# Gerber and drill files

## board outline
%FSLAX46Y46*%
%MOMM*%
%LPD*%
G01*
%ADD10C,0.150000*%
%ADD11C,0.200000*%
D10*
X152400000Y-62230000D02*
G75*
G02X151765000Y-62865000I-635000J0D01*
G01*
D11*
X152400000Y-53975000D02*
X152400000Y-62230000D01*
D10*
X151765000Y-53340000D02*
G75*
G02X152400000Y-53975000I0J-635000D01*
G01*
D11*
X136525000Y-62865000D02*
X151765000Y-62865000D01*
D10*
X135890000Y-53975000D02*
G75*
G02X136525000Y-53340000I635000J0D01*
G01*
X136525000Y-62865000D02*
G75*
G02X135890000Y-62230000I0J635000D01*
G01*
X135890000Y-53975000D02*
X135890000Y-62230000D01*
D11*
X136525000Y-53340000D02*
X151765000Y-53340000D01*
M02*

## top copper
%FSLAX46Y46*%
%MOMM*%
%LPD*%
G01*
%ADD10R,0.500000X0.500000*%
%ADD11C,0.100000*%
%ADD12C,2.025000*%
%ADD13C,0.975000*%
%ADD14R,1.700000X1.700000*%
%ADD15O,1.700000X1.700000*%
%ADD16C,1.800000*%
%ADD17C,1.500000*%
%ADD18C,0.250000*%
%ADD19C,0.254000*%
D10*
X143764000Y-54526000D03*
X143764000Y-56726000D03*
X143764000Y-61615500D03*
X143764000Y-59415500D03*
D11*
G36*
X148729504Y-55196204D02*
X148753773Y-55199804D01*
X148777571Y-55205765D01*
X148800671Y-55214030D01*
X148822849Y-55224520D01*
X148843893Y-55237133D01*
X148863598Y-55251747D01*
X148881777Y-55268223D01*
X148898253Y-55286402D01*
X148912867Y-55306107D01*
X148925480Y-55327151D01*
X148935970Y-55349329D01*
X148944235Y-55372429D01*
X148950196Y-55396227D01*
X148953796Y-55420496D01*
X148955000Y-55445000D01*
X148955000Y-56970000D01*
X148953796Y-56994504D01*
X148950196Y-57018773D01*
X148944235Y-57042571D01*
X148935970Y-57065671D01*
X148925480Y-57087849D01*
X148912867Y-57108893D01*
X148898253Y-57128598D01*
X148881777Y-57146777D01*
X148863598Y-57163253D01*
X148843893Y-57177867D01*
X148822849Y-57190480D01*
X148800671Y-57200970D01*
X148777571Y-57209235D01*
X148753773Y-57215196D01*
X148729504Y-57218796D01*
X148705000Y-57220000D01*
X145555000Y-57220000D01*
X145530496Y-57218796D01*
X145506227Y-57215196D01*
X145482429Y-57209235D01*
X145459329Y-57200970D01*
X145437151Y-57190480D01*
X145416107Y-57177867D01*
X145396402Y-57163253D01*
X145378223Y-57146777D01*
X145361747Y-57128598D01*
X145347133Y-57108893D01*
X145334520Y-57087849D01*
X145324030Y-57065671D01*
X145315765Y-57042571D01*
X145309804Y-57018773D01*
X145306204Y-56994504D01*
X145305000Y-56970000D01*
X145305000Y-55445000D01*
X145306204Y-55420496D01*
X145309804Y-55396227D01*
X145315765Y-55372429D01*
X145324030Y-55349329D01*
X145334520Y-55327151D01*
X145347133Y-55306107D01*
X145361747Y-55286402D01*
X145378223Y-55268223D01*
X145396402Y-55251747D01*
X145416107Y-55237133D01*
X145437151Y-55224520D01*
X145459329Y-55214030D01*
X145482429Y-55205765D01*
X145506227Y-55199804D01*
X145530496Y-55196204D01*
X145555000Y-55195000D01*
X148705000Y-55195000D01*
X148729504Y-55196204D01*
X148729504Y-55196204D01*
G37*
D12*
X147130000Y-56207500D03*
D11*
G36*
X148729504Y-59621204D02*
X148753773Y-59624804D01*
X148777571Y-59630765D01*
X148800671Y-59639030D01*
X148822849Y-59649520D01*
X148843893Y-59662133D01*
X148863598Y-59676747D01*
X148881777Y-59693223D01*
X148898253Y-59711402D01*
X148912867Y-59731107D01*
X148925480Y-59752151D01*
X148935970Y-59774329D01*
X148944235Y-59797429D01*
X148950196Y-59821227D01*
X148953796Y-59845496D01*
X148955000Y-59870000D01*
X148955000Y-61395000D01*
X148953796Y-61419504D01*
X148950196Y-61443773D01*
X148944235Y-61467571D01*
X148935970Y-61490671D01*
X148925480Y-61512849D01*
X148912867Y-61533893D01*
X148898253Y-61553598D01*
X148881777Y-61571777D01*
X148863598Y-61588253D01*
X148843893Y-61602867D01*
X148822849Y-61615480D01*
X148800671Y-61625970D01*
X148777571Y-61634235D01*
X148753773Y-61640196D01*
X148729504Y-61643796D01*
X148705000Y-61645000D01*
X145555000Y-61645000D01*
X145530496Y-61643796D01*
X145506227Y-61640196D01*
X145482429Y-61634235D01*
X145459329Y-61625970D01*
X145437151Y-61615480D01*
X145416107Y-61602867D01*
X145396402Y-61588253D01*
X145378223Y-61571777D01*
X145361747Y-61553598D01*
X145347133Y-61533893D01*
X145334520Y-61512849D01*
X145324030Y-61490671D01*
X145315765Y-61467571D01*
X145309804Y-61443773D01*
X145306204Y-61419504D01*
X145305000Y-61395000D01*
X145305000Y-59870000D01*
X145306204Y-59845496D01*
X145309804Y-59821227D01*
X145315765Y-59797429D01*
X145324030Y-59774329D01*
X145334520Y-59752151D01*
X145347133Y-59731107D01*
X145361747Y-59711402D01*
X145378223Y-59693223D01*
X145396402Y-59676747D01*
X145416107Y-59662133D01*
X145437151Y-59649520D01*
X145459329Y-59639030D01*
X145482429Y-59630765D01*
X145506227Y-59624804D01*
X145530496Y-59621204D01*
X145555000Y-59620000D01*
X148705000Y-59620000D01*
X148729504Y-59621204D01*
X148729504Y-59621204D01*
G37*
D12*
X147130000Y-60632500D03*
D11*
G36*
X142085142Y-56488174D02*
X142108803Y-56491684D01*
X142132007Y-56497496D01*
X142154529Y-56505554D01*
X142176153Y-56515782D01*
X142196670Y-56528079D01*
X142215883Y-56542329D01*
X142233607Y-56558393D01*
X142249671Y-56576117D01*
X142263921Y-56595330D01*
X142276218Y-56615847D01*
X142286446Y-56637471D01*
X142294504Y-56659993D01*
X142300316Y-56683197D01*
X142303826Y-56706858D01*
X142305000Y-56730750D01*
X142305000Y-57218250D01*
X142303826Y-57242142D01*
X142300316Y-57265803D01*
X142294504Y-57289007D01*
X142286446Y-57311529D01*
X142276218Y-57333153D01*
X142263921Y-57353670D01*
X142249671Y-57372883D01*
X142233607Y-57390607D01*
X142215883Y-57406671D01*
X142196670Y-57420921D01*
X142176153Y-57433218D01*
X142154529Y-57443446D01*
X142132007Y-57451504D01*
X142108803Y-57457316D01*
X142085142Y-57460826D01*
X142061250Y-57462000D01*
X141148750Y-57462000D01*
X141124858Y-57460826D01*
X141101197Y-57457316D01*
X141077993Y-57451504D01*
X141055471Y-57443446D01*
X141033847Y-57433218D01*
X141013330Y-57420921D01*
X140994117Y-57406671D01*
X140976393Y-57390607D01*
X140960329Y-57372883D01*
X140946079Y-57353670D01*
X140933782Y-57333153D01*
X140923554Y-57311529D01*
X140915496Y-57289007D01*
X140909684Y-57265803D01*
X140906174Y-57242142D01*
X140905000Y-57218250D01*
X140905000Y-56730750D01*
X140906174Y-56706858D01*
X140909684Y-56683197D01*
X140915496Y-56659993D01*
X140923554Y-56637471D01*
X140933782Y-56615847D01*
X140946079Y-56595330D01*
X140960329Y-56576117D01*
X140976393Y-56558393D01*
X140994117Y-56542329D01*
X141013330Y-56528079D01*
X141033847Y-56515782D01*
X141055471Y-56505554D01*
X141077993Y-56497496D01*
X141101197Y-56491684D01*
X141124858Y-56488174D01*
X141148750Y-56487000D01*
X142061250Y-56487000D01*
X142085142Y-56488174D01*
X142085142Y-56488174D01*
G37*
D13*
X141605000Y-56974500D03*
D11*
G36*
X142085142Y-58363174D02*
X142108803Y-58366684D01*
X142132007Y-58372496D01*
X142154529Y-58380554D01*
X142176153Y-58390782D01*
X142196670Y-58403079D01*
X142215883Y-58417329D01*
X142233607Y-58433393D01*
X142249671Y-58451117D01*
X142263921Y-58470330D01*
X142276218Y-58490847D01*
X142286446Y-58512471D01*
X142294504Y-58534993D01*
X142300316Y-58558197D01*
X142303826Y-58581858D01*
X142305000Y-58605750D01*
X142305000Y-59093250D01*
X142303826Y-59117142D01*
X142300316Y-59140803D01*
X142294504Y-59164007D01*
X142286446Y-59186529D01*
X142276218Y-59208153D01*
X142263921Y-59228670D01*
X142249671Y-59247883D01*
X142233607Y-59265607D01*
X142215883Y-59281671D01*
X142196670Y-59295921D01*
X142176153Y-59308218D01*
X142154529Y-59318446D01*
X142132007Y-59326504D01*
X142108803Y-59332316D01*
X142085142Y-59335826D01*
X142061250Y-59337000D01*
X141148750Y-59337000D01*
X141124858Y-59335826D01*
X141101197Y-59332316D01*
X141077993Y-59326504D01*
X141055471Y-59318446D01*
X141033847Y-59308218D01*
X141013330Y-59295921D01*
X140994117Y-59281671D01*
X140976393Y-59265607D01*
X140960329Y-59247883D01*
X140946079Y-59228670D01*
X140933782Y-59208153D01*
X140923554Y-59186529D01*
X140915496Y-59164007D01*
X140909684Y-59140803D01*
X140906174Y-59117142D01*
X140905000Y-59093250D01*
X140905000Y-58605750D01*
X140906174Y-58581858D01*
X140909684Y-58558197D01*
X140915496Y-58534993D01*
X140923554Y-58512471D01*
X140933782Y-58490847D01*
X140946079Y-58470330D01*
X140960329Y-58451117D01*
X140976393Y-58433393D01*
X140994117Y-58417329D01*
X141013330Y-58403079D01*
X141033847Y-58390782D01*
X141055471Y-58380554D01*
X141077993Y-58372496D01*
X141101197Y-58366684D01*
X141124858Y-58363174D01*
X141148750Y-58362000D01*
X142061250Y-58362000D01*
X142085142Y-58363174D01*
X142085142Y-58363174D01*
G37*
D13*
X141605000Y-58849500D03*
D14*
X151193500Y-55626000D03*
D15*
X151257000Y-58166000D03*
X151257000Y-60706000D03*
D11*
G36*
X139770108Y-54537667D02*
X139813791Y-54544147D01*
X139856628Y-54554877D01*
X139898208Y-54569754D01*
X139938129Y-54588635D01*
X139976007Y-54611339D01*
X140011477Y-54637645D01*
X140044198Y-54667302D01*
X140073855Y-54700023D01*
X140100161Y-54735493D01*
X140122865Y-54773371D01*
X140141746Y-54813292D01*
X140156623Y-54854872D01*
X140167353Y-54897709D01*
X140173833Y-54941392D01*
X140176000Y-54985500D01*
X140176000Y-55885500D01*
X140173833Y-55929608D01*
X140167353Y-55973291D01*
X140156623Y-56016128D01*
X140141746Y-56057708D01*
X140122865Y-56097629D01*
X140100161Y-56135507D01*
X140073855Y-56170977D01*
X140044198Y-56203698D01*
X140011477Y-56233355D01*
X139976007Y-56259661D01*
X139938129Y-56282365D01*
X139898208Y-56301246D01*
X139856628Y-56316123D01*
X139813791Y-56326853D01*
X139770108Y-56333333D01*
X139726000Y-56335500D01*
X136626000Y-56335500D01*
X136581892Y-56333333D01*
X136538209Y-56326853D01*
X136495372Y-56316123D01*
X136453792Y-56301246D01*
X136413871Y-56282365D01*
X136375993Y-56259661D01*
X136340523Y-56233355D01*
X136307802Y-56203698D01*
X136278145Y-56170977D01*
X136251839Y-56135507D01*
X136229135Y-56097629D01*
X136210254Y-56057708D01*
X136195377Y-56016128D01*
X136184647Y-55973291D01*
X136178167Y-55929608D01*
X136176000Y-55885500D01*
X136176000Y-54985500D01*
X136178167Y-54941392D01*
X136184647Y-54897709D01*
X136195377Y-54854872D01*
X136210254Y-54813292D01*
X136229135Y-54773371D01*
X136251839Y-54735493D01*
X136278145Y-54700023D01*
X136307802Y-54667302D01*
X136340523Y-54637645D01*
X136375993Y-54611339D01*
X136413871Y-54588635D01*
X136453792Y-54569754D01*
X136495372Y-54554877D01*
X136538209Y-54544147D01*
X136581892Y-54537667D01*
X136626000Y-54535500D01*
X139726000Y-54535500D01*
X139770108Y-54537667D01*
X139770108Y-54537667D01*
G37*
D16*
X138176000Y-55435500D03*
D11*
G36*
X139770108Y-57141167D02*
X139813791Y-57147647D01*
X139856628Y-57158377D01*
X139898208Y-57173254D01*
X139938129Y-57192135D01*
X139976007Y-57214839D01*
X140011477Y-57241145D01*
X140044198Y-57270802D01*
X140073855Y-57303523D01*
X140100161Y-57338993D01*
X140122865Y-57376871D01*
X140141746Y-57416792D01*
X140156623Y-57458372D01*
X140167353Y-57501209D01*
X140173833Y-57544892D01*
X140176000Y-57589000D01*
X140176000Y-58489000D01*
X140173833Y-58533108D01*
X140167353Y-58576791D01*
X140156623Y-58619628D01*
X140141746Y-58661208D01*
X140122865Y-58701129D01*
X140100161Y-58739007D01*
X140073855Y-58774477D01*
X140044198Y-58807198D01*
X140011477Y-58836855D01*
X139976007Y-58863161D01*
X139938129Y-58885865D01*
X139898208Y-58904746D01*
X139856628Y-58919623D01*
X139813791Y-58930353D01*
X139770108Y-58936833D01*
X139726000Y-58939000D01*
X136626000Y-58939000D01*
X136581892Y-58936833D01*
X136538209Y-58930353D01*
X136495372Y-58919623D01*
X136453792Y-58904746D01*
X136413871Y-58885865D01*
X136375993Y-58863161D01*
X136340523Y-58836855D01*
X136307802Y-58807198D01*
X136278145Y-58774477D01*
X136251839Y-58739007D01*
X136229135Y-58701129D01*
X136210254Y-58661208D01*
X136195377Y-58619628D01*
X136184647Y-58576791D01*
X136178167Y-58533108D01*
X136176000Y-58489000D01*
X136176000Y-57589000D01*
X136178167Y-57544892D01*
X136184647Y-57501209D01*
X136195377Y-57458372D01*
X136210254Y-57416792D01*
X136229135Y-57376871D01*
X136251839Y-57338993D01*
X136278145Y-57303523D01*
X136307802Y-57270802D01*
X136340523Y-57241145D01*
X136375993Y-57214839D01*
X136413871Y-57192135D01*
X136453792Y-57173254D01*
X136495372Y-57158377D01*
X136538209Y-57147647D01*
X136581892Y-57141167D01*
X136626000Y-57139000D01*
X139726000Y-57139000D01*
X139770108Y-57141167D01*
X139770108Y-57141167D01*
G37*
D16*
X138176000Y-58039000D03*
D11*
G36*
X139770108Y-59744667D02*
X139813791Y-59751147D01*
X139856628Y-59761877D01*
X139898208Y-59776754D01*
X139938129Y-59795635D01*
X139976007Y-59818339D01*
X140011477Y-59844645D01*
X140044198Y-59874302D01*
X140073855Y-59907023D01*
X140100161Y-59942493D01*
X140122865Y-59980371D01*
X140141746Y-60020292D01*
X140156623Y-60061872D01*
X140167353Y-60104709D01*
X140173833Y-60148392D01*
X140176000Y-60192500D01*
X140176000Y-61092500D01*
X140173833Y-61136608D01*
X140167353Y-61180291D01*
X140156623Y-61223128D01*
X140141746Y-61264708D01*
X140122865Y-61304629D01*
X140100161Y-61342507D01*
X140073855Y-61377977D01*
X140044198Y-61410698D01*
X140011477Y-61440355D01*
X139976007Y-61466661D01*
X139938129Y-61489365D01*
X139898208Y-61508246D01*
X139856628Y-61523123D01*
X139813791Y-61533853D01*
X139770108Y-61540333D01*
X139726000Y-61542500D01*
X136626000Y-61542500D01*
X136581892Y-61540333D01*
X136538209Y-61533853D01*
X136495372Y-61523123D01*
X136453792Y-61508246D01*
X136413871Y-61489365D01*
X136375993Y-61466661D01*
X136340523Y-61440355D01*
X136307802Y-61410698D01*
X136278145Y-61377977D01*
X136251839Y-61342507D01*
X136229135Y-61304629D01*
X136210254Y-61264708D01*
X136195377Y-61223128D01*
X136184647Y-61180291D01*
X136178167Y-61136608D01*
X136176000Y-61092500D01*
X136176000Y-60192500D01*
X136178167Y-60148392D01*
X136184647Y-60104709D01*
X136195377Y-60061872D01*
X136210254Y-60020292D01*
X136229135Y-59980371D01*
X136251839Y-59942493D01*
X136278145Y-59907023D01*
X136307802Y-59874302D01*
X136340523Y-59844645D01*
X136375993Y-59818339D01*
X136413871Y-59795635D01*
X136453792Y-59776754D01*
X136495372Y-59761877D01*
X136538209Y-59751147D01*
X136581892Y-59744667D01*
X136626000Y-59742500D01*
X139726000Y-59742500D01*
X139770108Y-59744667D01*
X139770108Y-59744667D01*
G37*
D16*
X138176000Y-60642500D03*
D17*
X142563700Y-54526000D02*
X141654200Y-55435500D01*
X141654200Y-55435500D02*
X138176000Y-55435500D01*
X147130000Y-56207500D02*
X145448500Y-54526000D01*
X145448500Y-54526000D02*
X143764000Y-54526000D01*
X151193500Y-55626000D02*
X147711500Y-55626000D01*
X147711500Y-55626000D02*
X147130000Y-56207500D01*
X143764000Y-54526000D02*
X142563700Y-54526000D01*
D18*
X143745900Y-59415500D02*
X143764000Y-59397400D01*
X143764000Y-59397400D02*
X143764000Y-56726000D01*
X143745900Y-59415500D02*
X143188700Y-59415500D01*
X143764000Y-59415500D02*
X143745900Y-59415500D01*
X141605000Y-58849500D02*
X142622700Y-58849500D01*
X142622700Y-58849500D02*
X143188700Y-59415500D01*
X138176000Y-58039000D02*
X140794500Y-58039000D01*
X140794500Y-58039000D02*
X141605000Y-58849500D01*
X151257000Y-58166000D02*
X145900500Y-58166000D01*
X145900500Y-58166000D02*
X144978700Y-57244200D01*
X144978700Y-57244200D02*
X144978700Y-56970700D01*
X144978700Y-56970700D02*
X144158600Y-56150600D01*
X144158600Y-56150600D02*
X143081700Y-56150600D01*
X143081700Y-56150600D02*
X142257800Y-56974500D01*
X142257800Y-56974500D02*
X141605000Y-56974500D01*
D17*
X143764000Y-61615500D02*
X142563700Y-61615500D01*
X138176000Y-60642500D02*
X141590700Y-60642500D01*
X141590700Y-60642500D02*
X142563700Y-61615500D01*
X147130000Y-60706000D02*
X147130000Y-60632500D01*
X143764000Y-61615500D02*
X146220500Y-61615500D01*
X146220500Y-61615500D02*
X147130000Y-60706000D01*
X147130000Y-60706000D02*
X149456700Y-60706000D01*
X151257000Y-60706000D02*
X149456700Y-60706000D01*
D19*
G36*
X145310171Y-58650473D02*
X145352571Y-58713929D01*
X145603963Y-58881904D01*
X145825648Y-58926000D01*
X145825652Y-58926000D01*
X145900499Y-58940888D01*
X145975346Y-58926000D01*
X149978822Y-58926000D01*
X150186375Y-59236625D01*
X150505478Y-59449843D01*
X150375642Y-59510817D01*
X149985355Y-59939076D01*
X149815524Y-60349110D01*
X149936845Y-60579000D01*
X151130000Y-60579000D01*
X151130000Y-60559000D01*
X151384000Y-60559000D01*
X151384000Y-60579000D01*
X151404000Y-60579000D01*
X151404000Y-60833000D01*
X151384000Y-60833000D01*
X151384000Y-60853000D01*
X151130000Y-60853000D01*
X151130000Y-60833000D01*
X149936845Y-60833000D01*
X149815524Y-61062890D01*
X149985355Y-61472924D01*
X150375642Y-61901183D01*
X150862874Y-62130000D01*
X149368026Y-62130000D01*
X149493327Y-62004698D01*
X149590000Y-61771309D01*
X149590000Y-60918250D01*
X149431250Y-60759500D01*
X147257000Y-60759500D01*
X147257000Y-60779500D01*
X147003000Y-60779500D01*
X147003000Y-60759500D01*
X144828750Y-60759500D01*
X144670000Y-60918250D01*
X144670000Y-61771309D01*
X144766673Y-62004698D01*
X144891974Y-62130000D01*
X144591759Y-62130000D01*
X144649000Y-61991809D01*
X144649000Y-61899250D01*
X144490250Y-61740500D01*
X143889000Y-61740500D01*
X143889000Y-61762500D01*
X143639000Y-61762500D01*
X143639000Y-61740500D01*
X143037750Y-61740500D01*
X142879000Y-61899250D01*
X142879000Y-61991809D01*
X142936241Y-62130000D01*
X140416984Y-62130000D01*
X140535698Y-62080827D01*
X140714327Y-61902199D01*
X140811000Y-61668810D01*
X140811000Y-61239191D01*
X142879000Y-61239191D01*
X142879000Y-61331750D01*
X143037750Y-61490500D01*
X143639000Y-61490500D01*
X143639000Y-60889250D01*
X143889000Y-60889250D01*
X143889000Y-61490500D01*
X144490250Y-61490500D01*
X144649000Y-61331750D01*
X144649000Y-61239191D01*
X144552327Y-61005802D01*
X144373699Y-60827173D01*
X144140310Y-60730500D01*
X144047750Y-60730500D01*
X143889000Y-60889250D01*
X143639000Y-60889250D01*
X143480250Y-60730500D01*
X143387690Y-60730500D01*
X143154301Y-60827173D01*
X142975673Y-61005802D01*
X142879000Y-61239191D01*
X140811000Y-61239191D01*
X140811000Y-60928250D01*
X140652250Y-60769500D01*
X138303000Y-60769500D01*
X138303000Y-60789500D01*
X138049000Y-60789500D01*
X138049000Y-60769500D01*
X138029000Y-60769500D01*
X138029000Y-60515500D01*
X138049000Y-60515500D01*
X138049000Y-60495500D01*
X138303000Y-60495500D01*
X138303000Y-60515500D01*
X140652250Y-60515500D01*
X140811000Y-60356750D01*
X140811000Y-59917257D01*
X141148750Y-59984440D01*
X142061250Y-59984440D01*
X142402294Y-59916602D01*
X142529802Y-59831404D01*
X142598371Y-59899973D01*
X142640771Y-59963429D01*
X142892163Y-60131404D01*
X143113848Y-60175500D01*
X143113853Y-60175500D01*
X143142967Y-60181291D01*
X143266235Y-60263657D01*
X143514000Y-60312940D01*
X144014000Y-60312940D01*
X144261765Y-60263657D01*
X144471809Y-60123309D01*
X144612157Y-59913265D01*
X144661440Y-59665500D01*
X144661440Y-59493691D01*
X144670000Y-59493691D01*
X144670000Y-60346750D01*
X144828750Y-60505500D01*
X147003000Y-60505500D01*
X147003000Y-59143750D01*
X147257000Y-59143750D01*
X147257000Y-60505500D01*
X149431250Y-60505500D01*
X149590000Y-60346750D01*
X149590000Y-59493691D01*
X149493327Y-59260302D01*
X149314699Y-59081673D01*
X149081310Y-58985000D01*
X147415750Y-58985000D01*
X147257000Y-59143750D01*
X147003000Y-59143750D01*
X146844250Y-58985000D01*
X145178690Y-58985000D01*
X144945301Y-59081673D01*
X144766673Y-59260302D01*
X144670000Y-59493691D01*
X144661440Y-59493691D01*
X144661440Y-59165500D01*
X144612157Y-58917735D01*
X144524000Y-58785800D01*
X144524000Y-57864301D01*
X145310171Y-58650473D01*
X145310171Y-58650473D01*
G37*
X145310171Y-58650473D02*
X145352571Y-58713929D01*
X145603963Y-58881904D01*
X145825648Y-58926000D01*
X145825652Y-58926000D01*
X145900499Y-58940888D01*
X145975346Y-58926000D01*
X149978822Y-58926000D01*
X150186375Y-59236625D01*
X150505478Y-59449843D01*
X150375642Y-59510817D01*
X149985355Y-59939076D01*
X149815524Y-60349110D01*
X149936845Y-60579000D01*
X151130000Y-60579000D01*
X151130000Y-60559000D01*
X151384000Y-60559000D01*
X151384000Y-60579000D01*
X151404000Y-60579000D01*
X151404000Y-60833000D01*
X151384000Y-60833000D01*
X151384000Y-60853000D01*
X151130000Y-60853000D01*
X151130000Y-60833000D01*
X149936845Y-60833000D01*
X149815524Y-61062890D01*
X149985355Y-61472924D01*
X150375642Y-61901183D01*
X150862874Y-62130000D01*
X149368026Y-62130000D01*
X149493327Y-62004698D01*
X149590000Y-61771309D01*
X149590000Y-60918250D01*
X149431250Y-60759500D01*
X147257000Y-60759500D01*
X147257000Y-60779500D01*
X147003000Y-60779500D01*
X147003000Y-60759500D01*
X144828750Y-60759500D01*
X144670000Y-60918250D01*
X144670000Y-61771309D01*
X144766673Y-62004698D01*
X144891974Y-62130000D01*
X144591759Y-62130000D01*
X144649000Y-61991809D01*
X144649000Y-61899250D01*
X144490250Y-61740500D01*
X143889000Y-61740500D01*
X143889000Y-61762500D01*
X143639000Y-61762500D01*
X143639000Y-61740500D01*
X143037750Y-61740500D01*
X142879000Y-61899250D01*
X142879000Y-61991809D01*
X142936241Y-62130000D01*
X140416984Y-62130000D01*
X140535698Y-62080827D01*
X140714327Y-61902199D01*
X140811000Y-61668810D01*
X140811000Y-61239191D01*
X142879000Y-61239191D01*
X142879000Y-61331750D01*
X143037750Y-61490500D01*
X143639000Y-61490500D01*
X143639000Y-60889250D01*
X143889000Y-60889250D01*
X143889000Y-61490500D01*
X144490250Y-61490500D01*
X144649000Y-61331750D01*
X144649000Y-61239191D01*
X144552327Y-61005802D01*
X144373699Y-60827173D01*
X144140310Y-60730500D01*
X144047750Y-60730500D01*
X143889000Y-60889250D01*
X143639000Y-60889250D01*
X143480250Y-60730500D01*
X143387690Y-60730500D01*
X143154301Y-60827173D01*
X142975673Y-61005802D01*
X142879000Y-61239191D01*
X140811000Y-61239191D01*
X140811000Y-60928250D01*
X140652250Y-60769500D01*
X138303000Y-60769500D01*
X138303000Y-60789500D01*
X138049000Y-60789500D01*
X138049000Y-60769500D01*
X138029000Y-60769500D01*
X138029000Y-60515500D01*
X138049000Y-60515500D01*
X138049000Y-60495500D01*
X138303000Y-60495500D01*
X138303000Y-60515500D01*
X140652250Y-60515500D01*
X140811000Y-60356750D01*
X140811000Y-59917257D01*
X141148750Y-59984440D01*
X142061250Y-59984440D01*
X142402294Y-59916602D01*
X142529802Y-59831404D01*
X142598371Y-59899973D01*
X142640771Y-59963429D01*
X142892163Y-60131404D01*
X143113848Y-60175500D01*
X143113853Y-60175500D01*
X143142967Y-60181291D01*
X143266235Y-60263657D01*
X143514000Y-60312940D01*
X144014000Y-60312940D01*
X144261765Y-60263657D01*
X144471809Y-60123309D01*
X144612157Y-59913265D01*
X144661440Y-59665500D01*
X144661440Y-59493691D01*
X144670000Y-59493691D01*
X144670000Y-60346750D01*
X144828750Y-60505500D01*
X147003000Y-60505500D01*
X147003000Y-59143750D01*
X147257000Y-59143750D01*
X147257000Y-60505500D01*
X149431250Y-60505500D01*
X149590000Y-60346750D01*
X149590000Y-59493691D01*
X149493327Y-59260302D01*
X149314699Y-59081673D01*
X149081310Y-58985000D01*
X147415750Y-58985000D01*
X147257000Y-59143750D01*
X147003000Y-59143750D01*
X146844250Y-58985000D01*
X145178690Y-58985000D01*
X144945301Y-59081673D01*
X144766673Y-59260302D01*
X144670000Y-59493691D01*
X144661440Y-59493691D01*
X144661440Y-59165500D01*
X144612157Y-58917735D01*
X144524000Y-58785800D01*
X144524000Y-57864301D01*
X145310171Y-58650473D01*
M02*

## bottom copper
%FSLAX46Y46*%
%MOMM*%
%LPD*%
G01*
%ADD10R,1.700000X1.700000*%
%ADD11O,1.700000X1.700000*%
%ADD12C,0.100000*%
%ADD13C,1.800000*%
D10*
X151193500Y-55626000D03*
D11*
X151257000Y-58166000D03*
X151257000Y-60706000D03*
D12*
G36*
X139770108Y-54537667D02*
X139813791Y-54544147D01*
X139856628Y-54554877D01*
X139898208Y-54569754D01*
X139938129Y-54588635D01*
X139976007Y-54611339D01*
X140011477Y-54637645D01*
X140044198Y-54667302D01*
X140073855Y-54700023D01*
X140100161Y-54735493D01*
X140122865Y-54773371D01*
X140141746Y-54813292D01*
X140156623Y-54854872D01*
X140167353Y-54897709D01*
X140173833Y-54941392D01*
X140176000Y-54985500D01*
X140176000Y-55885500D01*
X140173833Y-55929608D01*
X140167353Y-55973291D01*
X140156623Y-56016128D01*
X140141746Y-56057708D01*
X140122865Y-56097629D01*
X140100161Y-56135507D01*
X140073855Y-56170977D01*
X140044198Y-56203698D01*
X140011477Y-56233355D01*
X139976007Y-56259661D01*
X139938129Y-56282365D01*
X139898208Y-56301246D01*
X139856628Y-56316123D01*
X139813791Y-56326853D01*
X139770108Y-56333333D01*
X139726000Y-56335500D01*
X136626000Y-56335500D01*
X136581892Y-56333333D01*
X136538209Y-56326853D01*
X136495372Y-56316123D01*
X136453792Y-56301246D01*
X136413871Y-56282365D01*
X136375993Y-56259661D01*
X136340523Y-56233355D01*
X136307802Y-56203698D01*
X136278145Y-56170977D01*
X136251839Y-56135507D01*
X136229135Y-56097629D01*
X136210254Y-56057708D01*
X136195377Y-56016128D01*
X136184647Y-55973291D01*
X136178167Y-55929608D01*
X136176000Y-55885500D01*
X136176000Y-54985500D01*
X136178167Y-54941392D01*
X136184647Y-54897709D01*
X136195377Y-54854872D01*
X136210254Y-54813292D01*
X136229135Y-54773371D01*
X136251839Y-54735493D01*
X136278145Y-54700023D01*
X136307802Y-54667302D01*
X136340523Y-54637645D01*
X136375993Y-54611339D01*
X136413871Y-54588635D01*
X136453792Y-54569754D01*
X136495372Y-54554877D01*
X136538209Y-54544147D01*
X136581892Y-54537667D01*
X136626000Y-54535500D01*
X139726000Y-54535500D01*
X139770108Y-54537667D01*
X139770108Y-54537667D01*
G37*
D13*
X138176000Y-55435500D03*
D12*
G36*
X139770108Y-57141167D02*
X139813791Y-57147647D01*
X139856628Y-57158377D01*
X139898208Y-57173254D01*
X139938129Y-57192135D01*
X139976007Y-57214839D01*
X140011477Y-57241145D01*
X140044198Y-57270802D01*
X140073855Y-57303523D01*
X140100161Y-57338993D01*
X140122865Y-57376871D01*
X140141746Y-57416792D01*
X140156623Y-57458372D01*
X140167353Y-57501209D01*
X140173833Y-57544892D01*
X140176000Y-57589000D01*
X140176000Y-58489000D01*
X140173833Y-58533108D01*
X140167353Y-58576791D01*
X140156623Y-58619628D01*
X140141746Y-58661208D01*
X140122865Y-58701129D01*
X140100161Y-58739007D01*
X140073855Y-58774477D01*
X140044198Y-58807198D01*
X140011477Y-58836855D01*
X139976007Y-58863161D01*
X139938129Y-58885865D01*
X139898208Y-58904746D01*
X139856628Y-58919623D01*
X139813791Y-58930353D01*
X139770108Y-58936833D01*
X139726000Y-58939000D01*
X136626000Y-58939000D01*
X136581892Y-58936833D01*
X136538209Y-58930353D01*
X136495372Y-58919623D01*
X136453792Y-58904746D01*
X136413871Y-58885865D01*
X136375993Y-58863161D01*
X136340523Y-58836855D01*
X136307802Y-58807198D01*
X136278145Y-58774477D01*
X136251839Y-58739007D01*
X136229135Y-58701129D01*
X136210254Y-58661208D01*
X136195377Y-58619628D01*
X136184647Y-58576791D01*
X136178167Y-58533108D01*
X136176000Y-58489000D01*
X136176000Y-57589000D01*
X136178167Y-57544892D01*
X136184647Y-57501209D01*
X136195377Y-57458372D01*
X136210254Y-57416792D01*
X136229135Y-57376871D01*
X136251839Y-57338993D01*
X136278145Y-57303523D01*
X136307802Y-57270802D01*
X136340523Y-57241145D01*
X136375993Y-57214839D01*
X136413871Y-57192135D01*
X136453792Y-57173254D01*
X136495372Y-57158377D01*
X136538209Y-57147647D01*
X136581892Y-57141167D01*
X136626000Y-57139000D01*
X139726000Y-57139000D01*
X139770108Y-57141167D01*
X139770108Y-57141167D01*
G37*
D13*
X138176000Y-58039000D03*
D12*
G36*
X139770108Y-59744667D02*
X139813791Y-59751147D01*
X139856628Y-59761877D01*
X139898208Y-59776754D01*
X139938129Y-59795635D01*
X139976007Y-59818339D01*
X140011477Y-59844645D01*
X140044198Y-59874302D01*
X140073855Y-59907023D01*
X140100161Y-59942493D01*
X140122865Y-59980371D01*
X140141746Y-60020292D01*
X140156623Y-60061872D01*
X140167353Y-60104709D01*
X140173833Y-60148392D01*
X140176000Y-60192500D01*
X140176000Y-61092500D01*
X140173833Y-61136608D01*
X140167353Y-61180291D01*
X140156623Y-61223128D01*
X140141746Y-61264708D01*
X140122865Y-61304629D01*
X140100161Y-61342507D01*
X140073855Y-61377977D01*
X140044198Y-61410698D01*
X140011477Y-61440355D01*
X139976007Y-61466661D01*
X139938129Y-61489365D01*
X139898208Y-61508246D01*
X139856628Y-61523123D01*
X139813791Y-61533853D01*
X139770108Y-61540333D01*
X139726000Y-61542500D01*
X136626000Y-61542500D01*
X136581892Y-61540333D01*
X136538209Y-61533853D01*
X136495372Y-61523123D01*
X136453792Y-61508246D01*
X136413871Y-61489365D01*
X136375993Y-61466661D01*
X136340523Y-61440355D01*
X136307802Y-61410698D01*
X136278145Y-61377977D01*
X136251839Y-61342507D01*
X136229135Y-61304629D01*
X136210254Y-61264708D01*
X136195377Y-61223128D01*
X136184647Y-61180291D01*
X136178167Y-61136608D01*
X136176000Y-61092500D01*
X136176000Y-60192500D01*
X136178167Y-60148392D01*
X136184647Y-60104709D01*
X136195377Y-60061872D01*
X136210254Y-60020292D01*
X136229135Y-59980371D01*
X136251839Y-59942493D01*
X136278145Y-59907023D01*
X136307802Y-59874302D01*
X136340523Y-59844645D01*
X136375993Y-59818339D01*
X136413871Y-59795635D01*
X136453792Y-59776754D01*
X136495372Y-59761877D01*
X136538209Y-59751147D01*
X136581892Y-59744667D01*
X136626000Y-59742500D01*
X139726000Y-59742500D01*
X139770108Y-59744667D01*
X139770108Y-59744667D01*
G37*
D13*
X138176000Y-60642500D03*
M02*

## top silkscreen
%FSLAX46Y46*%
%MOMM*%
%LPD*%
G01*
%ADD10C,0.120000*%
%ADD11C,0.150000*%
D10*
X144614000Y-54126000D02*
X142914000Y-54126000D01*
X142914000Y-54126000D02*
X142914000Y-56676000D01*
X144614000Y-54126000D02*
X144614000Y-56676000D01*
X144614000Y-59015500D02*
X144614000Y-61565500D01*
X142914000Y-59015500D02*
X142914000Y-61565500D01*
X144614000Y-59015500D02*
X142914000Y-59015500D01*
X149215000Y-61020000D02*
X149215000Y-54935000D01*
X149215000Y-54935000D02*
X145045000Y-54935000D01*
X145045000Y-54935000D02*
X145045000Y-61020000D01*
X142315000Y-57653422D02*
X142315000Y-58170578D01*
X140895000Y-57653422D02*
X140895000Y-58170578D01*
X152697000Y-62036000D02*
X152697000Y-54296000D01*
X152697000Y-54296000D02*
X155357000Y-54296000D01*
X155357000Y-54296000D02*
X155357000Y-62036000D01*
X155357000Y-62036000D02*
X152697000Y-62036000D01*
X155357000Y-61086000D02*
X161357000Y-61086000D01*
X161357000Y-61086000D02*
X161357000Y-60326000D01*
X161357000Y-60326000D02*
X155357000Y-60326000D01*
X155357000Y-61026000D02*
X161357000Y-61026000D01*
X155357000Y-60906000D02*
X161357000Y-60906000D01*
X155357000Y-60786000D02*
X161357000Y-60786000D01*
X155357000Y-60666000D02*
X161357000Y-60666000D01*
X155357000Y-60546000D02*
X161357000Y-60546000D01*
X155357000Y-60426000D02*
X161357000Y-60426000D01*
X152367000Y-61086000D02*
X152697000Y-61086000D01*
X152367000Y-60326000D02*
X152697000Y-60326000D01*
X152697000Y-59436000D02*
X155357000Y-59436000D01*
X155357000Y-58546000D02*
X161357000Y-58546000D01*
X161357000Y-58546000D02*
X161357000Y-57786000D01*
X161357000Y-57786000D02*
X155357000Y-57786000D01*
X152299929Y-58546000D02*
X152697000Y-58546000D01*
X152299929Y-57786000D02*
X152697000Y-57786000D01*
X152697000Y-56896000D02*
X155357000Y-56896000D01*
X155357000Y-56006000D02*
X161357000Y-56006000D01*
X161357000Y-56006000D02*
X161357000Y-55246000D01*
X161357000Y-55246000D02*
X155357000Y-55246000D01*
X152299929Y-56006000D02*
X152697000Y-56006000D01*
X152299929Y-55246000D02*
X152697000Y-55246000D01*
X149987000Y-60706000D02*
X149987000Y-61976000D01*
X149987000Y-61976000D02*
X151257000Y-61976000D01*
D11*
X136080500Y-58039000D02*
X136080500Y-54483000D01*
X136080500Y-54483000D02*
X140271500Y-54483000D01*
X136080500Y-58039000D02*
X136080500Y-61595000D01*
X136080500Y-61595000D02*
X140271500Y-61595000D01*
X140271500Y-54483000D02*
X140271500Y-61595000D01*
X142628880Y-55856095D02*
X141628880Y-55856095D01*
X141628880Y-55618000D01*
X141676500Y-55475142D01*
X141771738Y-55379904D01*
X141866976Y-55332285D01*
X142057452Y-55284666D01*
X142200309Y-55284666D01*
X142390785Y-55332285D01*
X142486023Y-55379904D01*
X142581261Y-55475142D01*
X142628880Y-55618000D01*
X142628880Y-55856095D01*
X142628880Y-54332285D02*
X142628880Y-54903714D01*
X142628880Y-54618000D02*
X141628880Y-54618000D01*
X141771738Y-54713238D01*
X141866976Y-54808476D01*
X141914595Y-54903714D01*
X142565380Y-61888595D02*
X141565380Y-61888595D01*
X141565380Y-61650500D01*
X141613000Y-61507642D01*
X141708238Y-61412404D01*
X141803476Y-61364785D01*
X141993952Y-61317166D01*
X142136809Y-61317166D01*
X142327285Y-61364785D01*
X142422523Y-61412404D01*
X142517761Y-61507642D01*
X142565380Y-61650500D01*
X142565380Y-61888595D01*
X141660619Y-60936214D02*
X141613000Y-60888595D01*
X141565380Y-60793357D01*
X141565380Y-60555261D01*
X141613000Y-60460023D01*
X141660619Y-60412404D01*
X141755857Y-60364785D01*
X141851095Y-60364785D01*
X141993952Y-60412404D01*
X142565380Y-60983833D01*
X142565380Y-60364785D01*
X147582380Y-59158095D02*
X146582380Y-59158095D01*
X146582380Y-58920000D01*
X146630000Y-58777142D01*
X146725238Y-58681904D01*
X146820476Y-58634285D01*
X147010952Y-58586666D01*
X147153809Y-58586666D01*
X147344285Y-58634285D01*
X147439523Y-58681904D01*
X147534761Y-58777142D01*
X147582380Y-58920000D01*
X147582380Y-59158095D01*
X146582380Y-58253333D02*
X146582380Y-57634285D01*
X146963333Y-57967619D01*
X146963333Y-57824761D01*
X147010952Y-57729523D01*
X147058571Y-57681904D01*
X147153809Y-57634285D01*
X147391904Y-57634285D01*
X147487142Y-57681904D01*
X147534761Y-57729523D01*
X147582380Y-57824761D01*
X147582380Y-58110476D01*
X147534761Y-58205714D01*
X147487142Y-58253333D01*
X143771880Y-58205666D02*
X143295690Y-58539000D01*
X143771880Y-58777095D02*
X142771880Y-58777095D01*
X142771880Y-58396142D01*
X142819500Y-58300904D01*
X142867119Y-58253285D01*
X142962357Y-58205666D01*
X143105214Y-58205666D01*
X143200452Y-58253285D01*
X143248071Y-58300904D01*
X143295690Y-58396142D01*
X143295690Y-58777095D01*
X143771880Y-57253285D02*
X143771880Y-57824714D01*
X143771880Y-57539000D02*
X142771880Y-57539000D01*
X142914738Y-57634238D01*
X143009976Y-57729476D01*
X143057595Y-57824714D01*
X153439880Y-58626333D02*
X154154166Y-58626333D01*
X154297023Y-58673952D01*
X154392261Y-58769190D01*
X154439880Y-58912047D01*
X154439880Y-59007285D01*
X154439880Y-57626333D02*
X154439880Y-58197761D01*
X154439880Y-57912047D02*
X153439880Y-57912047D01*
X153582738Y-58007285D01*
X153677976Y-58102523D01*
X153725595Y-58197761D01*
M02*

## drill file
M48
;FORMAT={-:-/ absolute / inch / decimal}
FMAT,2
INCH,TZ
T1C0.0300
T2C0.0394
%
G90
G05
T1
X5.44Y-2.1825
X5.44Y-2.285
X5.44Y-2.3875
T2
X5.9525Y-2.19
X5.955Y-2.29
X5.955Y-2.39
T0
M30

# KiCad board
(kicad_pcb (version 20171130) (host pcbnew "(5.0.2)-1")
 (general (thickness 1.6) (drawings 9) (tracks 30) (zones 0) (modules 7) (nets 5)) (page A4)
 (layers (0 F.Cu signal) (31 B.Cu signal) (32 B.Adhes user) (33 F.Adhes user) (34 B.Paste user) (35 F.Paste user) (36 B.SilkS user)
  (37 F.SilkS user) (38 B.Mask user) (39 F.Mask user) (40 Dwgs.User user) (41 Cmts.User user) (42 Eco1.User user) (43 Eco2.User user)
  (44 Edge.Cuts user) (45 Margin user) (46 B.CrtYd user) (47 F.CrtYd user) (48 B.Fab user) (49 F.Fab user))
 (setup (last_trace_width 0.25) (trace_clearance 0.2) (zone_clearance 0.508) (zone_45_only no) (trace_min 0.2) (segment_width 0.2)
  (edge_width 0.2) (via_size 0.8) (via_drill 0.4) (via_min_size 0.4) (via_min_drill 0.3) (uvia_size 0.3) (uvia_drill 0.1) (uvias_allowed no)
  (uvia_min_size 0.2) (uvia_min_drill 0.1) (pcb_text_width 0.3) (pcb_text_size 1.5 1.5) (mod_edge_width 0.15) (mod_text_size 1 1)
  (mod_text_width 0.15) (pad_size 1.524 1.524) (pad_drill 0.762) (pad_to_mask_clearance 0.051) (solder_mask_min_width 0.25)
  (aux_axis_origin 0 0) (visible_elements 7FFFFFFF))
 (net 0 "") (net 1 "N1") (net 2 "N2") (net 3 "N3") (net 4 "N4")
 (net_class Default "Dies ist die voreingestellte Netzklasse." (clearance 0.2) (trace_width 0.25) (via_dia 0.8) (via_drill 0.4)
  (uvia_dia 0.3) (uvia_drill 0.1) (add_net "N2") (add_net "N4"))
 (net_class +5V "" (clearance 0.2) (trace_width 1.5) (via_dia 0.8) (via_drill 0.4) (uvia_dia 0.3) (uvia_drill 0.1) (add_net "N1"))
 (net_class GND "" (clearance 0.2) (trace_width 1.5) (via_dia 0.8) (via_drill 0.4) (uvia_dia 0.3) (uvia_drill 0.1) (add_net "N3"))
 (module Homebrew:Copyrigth (layer F.Cu) (at 140.0175 56.0705)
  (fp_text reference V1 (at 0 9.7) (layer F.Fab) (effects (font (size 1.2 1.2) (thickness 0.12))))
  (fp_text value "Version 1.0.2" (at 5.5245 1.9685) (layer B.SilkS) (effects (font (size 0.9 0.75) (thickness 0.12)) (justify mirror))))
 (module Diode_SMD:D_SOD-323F (layer F.Cu) (at 143.764 55.626 270)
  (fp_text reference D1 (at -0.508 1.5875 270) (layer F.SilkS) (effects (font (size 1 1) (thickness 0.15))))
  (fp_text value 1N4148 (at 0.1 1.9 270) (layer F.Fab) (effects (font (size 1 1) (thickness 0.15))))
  (fp_line (start -1.5 -0.85) (end -1.5 0.85) (layer F.SilkS) (width 0.12))
  (fp_line (start -1.5 0.85) (end 1.05 0.85) (layer F.SilkS) (width 0.12))
  (fp_line (start -1.5 -0.85) (end 1.05 -0.85) (layer F.SilkS) (width 0.12))
  (pad 1 smd rect (at -1.1 0 270) (size 0.5 0.5) (layers F.Cu F.Paste F.Mask) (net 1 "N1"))
  (pad 2 smd rect (at 1.1 0 270) (size 0.5 0.5) (layers F.Cu F.Paste F.Mask) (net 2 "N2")))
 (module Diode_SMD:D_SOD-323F (layer F.Cu) (at 143.764 60.5155 270)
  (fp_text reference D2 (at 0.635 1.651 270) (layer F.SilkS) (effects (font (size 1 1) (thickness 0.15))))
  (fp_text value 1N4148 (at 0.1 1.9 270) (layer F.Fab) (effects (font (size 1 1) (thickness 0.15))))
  (fp_line (start -1.5 -0.85) (end 1.05 -0.85) (layer F.SilkS) (width 0.12))
  (fp_line (start -1.5 0.85) (end 1.05 0.85) (layer F.SilkS) (width 0.12))
  (fp_line (start -1.5 -0.85) (end -1.5 0.85) (layer F.SilkS) (width 0.12))
  (pad 2 smd rect (at 1.1 0 270) (size 0.5 0.5) (layers F.Cu F.Paste F.Mask) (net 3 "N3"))
  (pad 1 smd rect (at -1.1 0 270) (size 0.5 0.5) (layers F.Cu F.Paste F.Mask) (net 2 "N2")))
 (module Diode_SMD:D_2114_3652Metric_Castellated (layer F.Cu) (at 147.13 58.42 270)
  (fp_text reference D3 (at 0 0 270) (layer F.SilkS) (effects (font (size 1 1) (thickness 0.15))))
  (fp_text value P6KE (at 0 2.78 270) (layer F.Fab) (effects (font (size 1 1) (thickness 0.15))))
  (fp_line (start 2.6 -2.085) (end -3.485 -2.085) (layer F.SilkS) (width 0.12))
  (fp_line (start -3.485 -2.085) (end -3.485 2.085) (layer F.SilkS) (width 0.12))
  (fp_line (start -3.485 2.085) (end 2.6 2.085) (layer F.SilkS) (width 0.12))
  (pad 1 smd roundrect (at -2.2125 0 270) (size 2.025 3.65) (layers F.Cu F.Paste F.Mask) (roundrect_rratio 0.123457) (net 1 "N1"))
  (pad 2 smd roundrect (at 2.2125 0 270) (size 2.025 3.65) (layers F.Cu F.Paste F.Mask) (roundrect_rratio 0.123457) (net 3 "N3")))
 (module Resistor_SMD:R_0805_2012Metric (layer F.Cu) (at 141.605 57.912 270)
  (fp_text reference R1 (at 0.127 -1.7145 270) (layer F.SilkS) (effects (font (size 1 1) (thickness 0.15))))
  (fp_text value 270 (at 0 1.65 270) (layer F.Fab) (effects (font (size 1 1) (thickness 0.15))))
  (fp_line (start -0.258578 -0.71) (end 0.258578 -0.71) (layer F.SilkS) (width 0.12))
  (fp_line (start -0.258578 0.71) (end 0.258578 0.71) (layer F.SilkS) (width 0.12))
  (pad 1 smd roundrect (at -0.9375 0 270) (size 0.975 1.4) (layers F.Cu F.Paste F.Mask) (roundrect_rratio 0.25) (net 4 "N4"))
  (pad 2 smd roundrect (at 0.9375 0 270) (size 0.975 1.4) (layers F.Cu F.Paste F.Mask) (roundrect_rratio 0.25) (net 2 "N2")))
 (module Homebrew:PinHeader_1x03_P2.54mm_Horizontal (layer F.Cu) (at 152.654 58.166)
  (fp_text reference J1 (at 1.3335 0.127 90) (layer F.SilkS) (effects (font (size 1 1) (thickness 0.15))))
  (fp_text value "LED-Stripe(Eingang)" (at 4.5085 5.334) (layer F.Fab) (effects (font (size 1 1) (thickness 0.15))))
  (fp_line (start 0.043 3.87) (end 0.043 -3.87) (layer F.SilkS) (width 0.12))
  (fp_line (start 0.043 -3.87) (end 2.703 -3.87) (layer F.SilkS) (width 0.12))
  (fp_line (start 2.703 -3.87) (end 2.703 3.87) (layer F.SilkS) (width 0.12))
  (fp_line (start 2.703 3.87) (end 0.043 3.87) (layer F.SilkS) (width 0.12))
  (fp_line (start 2.703 2.92) (end 8.703 2.92) (layer F.SilkS) (width 0.12))
  (fp_line (start 8.703 2.92) (end 8.703 2.16) (layer F.SilkS) (width 0.12))
  (fp_line (start 8.703 2.16) (end 2.703 2.16) (layer F.SilkS) (width 0.12))
  (fp_line (start 2.703 2.86) (end 8.703 2.86) (layer F.SilkS) (width 0.12))
  (fp_line (start 2.703 2.74) (end 8.703 2.74) (layer F.SilkS) (width 0.12))
  (fp_line (start 2.703 2.62) (end 8.703 2.62) (layer F.SilkS) (width 0.12))
  (fp_line (start 2.703 2.5) (end 8.703 2.5) (layer F.SilkS) (width 0.12))
  (fp_line (start 2.703 2.38) (end 8.703 2.38) (layer F.SilkS) (width 0.12))
  (fp_line (start 2.703 2.26) (end 8.703 2.26) (layer F.SilkS) (width 0.12))
  (fp_line (start -0.287 2.92) (end 0.043 2.92) (layer F.SilkS) (width 0.12))
  (fp_line (start -0.287 2.16) (end 0.043 2.16) (layer F.SilkS) (width 0.12))
  (fp_line (start 0.043 1.27) (end 2.703 1.27) (layer F.SilkS) (width 0.12))
  (fp_line (start 2.703 0.38) (end 8.703 0.38) (layer F.SilkS) (width 0.12))
  (fp_line (start 8.703 0.38) (end 8.703 -0.38) (layer F.SilkS) (width 0.12))
  (fp_line (start 8.703 -0.38) (end 2.703 -0.38) (layer F.SilkS) (width 0.12))
  (fp_line (start -0.354071 0.38) (end 0.043 0.38) (layer F.SilkS) (width 0.12))
  (fp_line (start -0.354071 -0.38) (end 0.043 -0.38) (layer F.SilkS) (width 0.12))
  (fp_line (start 0.043 -1.27) (end 2.703 -1.27) (layer F.SilkS) (width 0.12))
  (fp_line (start 2.703 -2.16) (end 8.703 -2.16) (layer F.SilkS) (width 0.12))
  (fp_line (start 8.703 -2.16) (end 8.703 -2.92) (layer F.SilkS) (width 0.12))
  (fp_line (start 8.703 -2.92) (end 2.703 -2.92) (layer F.SilkS) (width 0.12))
  (fp_line (start -0.354071 -2.16) (end 0.043 -2.16) (layer F.SilkS) (width 0.12))
  (fp_line (start -0.354071 -2.92) (end 0.043 -2.92) (layer F.SilkS) (width 0.12))
  (fp_line (start -2.667 2.54) (end -2.667 3.81) (layer F.SilkS) (width 0.12))
  (fp_line (start -2.667 3.81) (end -1.397 3.81) (layer F.SilkS) (width 0.12))
  (pad 1 thru_hole rect (at -1.4605 -2.54 180) (size 1.7 1.7) (drill 1) (layers *.Cu *.Mask) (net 1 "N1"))
  (pad 2 thru_hole oval (at -1.397 0 180) (size 1.7 1.7) (drill 1) (layers *.Cu *.Mask) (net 4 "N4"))
  (pad 3 thru_hole oval (at -1.397 2.54 180) (size 1.7 1.7) (drill 1) (layers *.Cu *.Mask) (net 3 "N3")))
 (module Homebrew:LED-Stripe (layer F.Cu) (at 138.176 57.9755)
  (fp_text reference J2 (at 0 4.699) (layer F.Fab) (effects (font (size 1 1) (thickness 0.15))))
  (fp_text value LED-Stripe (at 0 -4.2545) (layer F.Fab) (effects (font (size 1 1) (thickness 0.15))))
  (fp_line (start -2.0955 0.0635) (end -2.0955 -3.4925) (layer F.SilkS) (width 0.15))
  (fp_line (start -2.0955 -3.4925) (end 2.0955 -3.4925) (layer F.SilkS) (width 0.15))
  (fp_line (start -2.0955 0.0635) (end -2.0955 3.6195) (layer F.SilkS) (width 0.15))
  (fp_line (start -2.0955 3.6195) (end 2.0955 3.6195) (layer F.SilkS) (width 0.15))
  (fp_line (start 2.0955 -3.4925) (end 2.0955 3.6195) (layer F.SilkS) (width 0.15))
  (pad 1 thru_hole roundrect (at 0 -2.54) (size 4 1.8) (drill 0.762) (layers *.Cu *.Mask) (roundrect_rratio 0.25) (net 1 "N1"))
  (pad 2 thru_hole roundrect (at 0 0.0635) (size 4 1.8) (drill 0.762) (layers *.Cu *.Mask) (roundrect_rratio 0.25) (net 2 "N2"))
  (pad 3 thru_hole roundrect (at 0 2.667) (size 4 1.8) (drill 0.762) (layers *.Cu *.Mask) (roundrect_rratio 0.25) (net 3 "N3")))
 (gr_arc (start 151.765 62.23) (end 151.765 62.865) (angle -90) (layer Edge.Cuts) (width 0.15))
 (gr_line (start 152.4 53.975) (end 152.4 62.23) (layer Edge.Cuts) (width 0.2))
 (gr_arc (start 151.765 53.975) (end 152.4 53.975) (angle -90) (layer Edge.Cuts) (width 0.15))
 (gr_line (start 136.525 62.865) (end 151.765 62.865) (layer Edge.Cuts) (width 0.2))
 (gr_arc (start 136.525 53.975) (end 136.525 53.34) (angle -90) (layer Edge.Cuts) (width 0.15))
 (gr_arc (start 136.525 62.23) (end 135.89 62.23) (angle -90) (layer Edge.Cuts) (width 0.15))
 (gr_line (start 135.89 53.975) (end 135.89 62.23) (layer Edge.Cuts) (width 0.15))
 (gr_line (start 136.525 53.34) (end 151.765 53.34) (layer Edge.Cuts) (width 0.2))
 (segment (start 142.5637 54.526) (end 141.6542 55.4355) (width 1.5) (layer F.Cu) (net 1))
 (segment (start 141.6542 55.4355) (end 138.176 55.4355) (width 1.5) (layer F.Cu) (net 1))
 (segment (start 147.13 56.2075) (end 145.4485 54.526) (width 1.5) (layer F.Cu) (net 1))
 (segment (start 145.4485 54.526) (end 143.764 54.526) (width 1.5) (layer F.Cu) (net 1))
 (segment (start 151.1935 55.626) (end 147.7115 55.626) (width 1.5) (layer F.Cu) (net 1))
 (segment (start 147.7115 55.626) (end 147.13 56.2075) (width 1.5) (layer F.Cu) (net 1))
 (segment (start 143.764 54.526) (end 142.5637 54.526) (width 1.5) (layer F.Cu) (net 1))
 (segment (start 143.7459 59.4155) (end 143.764 59.3974) (width 0.25) (layer F.Cu) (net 2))
 (segment (start 143.764 59.3974) (end 143.764 56.726) (width 0.25) (layer F.Cu) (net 2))
 (segment (start 143.7459 59.4155) (end 143.1887 59.4155) (width 0.25) (layer F.Cu) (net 2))
 (segment (start 143.764 59.4155) (end 143.7459 59.4155) (width 0.25) (layer F.Cu) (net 2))
 (segment (start 141.605 58.8495) (end 142.6227 58.8495) (width 0.25) (layer F.Cu) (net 2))
 (segment (start 142.6227 58.8495) (end 143.1887 59.4155) (width 0.25) (layer F.Cu) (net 2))
 (segment (start 138.176 58.039) (end 140.7945 58.039) (width 0.25) (layer F.Cu) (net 2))
 (segment (start 140.7945 58.039) (end 141.605 58.8495) (width 0.25) (layer F.Cu) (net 2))
 (segment (start 151.257 58.166) (end 145.9005 58.166) (width 0.25) (layer F.Cu) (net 4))
 (segment (start 145.9005 58.166) (end 144.9787 57.2442) (width 0.25) (layer F.Cu) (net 4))
 (segment (start 144.9787 57.2442) (end 144.9787 56.9707) (width 0.25) (layer F.Cu) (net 4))
 (segment (start 144.9787 56.9707) (end 144.1586 56.1506) (width 0.25) (layer F.Cu) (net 4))
 (segment (start 144.1586 56.1506) (end 143.0817 56.1506) (width 0.25) (layer F.Cu) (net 4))
 (segment (start 143.0817 56.1506) (end 142.2578 56.9745) (width 0.25) (layer F.Cu) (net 4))
 (segment (start 142.2578 56.9745) (end 141.605 56.9745) (width 0.25) (layer F.Cu) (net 4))
 (segment (start 143.764 61.6155) (end 142.5637 61.6155) (width 1.5) (layer F.Cu) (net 3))
 (segment (start 138.176 60.6425) (end 141.5907 60.6425) (width 1.5) (layer F.Cu) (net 3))
 (segment (start 141.5907 60.6425) (end 142.5637 61.6155) (width 1.5) (layer F.Cu) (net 3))
 (segment (start 147.13 60.706) (end 147.13 60.6325) (width 1.5) (layer F.Cu) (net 3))
 (segment (start 143.764 61.6155) (end 146.2205 61.6155) (width 1.5) (layer F.Cu) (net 3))
 (segment (start 146.2205 61.6155) (end 147.13 60.706) (width 1.5) (layer F.Cu) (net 3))
 (segment (start 147.13 60.706) (end 149.4567 60.706) (width 1.5) (layer F.Cu) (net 3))
 (segment (start 151.257 60.706) (end 149.4567 60.706) (width 1.5) (layer F.Cu) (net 3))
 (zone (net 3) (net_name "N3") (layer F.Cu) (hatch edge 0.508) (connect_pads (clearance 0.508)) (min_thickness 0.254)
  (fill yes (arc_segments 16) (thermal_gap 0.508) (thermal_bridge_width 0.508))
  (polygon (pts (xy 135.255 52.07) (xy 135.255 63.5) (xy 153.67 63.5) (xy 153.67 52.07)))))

